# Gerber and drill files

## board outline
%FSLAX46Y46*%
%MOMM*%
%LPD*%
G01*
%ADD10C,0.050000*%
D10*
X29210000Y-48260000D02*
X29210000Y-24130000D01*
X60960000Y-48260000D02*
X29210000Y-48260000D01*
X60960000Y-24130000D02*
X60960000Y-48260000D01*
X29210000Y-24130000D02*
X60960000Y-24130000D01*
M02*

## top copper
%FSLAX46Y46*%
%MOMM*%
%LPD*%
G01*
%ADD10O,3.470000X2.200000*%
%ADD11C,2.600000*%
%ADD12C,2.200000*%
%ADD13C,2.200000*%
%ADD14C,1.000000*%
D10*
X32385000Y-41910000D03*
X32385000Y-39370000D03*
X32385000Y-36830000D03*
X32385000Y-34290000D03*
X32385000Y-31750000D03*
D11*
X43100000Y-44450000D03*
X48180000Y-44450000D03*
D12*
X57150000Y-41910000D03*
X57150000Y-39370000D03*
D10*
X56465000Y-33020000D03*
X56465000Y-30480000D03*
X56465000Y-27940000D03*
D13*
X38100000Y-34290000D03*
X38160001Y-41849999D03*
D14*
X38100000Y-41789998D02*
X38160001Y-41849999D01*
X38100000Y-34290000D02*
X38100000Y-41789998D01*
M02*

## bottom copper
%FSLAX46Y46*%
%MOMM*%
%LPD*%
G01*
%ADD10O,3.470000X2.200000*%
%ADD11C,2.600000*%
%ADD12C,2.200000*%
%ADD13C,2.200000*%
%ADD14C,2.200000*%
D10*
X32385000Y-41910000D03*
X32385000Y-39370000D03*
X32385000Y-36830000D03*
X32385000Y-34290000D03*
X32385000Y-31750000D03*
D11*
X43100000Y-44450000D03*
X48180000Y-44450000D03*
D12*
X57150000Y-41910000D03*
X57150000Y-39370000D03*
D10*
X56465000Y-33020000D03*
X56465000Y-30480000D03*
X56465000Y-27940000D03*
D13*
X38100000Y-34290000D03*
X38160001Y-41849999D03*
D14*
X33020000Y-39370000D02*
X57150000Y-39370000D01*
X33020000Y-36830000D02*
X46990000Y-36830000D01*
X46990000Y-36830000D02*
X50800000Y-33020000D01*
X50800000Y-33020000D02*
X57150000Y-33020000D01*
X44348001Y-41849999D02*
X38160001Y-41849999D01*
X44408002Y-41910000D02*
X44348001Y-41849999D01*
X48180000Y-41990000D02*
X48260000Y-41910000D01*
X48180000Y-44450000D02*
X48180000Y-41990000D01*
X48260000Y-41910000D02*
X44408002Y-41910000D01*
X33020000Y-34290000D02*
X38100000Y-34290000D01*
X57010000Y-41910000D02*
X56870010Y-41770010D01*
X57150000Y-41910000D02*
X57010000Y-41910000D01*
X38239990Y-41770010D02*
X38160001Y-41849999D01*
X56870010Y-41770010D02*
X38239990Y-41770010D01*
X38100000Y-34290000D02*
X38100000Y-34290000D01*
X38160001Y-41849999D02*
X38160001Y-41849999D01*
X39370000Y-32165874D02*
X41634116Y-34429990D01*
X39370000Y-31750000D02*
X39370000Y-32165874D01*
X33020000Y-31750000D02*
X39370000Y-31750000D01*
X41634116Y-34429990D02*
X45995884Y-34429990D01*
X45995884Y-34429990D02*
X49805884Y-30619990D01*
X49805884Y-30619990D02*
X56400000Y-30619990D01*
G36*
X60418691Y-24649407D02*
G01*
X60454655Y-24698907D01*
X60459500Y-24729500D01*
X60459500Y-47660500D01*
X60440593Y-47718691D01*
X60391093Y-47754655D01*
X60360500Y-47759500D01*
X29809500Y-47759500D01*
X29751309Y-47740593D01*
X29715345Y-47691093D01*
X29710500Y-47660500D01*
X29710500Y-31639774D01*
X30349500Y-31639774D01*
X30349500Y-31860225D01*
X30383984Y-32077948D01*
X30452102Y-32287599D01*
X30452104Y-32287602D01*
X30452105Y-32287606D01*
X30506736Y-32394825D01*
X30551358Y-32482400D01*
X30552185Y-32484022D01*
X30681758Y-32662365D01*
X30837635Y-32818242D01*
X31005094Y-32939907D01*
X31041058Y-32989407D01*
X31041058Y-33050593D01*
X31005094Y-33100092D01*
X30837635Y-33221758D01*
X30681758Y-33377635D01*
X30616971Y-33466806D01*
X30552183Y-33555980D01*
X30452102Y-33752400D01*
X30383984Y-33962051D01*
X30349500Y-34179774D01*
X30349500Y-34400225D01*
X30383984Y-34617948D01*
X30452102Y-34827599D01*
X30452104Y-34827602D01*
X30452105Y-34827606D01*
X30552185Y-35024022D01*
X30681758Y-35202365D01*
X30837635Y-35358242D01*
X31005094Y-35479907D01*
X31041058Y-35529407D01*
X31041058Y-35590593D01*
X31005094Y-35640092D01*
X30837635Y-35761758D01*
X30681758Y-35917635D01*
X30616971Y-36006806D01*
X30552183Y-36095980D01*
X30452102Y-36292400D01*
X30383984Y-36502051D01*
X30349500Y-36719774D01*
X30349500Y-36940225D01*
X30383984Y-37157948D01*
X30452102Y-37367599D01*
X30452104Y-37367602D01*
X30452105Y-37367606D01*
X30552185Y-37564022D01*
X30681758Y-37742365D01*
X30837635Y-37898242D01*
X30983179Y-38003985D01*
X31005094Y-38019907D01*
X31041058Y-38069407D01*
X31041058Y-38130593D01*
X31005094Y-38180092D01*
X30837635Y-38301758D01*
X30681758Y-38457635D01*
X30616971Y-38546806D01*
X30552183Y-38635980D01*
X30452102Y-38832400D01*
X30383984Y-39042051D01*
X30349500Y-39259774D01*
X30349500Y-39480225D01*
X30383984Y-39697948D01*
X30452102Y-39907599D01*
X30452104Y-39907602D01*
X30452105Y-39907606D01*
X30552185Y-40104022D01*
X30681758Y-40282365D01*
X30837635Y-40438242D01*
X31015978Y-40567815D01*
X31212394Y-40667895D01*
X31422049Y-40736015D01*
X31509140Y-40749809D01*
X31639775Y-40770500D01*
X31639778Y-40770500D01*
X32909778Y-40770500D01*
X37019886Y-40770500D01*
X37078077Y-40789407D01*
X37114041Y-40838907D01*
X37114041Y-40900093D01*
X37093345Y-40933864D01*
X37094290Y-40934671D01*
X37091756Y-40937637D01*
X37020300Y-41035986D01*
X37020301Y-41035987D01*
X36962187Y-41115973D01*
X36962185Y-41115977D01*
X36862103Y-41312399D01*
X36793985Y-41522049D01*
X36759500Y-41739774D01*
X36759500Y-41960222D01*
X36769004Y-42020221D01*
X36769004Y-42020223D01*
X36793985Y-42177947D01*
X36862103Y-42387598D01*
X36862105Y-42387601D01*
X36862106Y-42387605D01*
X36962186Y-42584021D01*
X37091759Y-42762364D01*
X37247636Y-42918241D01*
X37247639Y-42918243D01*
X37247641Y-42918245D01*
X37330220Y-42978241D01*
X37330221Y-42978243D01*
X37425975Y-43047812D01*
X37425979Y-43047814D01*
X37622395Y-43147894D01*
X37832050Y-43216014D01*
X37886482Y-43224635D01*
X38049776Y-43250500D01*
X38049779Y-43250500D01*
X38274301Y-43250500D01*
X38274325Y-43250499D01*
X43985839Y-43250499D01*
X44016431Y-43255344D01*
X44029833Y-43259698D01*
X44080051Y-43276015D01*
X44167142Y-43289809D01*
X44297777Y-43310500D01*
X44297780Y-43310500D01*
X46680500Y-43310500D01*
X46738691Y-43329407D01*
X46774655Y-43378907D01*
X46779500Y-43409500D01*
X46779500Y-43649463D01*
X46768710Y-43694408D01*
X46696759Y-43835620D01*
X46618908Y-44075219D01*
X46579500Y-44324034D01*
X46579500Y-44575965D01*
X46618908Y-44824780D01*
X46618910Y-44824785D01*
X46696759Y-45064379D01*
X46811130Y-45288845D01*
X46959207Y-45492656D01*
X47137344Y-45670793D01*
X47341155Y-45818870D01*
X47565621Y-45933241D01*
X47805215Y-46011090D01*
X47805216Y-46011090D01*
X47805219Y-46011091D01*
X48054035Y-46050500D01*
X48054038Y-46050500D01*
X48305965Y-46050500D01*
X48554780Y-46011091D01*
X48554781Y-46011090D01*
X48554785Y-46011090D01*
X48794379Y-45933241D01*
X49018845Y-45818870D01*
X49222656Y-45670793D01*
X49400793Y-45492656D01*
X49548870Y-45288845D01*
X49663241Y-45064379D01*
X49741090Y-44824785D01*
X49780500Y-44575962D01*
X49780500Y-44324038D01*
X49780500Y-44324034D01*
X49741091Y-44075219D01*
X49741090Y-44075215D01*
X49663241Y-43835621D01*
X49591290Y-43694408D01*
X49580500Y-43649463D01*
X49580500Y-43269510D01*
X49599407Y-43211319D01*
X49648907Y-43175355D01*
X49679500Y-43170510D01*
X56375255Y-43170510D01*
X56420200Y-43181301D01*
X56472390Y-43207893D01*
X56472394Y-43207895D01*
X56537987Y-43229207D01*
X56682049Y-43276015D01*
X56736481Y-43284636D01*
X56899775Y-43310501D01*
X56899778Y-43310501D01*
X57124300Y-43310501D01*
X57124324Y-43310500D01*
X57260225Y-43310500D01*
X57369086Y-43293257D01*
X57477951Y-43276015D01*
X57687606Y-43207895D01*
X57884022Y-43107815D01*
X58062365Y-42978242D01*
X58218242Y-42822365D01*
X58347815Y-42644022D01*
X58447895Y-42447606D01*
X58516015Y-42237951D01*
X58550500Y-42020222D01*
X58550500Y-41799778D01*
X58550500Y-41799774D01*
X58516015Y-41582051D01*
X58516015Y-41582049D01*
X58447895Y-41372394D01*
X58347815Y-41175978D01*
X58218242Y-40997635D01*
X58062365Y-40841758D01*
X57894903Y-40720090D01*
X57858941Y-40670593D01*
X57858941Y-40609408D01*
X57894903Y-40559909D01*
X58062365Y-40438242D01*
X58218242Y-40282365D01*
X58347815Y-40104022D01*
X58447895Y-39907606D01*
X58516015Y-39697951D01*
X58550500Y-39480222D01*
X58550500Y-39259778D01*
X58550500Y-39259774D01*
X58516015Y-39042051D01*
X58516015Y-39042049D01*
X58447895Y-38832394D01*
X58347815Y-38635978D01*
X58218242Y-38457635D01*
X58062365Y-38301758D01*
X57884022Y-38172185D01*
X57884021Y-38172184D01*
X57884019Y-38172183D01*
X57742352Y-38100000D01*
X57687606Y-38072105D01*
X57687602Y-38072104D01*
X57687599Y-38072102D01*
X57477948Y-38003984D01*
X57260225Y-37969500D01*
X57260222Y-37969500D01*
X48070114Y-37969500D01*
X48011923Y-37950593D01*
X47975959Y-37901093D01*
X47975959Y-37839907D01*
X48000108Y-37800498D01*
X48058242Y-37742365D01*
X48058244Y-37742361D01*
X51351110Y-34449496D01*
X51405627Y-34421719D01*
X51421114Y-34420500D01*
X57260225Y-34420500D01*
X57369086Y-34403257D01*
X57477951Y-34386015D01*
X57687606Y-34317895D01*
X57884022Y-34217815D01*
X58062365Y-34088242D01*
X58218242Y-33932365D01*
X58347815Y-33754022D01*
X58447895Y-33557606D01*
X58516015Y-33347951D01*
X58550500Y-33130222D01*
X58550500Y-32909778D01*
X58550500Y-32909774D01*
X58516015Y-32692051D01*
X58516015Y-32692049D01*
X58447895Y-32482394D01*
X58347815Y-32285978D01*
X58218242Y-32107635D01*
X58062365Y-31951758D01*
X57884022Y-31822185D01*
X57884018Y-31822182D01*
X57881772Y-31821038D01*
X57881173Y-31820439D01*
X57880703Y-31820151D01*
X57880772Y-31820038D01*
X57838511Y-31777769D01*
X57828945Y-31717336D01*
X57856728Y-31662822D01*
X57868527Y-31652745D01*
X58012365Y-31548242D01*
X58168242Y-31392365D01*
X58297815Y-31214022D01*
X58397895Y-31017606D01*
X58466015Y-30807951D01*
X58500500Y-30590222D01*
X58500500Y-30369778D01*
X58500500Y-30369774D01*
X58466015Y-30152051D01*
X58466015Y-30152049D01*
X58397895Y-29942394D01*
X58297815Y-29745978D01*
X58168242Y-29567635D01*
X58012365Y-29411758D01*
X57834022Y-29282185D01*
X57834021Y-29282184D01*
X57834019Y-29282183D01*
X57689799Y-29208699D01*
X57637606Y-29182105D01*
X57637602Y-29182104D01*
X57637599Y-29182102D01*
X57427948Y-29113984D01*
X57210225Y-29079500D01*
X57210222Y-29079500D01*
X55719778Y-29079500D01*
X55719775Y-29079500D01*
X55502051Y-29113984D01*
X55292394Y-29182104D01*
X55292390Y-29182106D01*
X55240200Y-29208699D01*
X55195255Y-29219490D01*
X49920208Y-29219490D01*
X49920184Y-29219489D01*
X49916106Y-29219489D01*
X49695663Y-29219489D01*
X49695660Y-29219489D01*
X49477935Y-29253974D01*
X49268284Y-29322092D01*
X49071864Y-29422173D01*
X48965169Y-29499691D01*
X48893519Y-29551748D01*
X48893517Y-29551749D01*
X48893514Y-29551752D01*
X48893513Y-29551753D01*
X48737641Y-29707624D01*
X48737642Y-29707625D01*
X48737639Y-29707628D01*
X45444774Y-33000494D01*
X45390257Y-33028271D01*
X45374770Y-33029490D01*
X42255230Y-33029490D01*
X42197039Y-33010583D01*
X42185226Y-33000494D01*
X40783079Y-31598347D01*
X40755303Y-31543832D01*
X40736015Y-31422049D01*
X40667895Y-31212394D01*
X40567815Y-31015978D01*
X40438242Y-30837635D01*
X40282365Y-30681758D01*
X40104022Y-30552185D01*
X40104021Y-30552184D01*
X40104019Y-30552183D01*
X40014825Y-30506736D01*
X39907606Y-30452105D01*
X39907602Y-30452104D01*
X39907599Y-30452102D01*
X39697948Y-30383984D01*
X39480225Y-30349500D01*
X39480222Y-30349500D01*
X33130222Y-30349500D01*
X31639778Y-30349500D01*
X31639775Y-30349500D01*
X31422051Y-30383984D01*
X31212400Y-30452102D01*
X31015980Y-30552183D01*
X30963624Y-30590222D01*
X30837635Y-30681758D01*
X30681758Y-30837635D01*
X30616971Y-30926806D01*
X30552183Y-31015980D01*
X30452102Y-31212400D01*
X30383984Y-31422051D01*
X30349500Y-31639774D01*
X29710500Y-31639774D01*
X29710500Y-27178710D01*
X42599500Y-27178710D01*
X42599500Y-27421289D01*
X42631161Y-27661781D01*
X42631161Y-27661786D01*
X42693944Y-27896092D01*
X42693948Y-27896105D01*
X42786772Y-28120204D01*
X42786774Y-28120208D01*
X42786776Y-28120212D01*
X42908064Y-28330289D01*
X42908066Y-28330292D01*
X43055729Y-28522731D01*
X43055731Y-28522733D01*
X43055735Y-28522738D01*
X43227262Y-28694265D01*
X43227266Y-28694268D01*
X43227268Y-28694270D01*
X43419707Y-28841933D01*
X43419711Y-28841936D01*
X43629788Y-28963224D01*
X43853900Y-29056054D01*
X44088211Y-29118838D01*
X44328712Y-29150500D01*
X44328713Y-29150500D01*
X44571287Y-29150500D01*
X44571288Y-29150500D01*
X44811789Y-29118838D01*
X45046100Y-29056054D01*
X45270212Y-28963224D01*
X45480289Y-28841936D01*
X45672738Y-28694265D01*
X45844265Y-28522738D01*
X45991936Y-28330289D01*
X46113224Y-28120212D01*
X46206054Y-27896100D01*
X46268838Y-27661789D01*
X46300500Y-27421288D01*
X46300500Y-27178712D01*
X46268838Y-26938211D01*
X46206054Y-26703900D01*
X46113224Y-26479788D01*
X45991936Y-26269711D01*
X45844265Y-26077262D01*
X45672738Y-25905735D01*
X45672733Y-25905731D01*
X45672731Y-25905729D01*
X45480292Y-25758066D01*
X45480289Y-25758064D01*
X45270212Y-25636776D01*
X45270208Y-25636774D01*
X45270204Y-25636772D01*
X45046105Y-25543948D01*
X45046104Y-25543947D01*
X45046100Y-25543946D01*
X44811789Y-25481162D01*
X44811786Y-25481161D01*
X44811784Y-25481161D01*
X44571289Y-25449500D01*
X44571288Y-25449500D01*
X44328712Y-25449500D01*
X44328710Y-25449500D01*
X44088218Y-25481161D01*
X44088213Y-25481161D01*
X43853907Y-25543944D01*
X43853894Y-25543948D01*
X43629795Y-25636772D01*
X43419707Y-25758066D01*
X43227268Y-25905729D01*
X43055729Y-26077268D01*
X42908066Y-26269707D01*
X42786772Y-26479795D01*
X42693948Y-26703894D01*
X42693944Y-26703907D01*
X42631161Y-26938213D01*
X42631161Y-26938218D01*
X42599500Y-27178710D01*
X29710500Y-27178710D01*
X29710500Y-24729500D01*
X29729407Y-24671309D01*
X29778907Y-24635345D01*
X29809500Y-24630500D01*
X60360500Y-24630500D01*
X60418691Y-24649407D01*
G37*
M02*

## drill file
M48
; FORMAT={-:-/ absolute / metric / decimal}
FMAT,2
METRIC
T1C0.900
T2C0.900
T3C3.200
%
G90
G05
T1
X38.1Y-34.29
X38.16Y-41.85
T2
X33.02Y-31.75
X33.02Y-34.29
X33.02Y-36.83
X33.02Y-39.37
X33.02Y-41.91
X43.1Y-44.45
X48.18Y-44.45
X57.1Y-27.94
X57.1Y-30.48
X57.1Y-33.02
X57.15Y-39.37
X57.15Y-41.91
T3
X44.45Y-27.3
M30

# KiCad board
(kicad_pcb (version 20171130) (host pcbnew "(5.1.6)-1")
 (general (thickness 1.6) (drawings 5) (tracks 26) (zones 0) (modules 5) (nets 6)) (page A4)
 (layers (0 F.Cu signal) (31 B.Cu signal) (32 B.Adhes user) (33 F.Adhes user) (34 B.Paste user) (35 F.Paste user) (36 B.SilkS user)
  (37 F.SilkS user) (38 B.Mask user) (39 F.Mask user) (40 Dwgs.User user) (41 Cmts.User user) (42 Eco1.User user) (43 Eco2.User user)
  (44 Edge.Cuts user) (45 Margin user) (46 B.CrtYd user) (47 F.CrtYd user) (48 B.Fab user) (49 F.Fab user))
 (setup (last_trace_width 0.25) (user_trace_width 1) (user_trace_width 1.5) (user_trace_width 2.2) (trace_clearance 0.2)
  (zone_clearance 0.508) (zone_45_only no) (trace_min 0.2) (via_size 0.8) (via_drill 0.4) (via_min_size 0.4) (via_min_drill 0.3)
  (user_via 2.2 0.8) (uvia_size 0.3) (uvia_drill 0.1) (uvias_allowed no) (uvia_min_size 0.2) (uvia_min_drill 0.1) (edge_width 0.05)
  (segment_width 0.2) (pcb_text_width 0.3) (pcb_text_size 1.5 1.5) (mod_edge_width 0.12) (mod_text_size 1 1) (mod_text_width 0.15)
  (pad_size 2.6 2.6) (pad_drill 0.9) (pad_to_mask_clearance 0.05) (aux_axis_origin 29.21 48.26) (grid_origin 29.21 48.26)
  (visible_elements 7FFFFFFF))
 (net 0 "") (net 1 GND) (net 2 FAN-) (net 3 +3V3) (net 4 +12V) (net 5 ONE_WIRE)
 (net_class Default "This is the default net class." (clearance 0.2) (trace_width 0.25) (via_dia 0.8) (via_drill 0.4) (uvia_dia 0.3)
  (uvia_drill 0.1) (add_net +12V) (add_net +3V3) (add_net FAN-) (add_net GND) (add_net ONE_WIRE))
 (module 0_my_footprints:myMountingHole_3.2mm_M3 (layer F.Cu) (at 44.45 27.3)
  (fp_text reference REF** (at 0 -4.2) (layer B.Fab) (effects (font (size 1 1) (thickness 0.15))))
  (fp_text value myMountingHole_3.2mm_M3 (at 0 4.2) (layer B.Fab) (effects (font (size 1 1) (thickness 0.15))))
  (pad "" np_thru_hole circle (at 0 0) (size 3.2 3.2) (drill 3.2) (layers *.Cu *.Mask)))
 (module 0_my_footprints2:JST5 (layer F.Cu) (at 33.02 41.91 90)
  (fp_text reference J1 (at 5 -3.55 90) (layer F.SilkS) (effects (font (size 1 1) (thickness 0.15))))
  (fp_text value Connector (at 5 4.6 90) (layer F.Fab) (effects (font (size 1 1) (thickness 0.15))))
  (pad 1 thru_hole oval (at 0 0 90) (size 2.2 3.47) (drill 0.9 (offset 0 -0.635)) (layers *.Cu *.Mask) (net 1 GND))
  (pad 2 thru_hole oval (at 2.54 0 90) (size 2.2 3.47) (drill 0.9 (offset 0 -0.635)) (layers *.Cu *.Mask) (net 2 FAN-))
  (pad 3 thru_hole oval (at 5.08 0 90) (size 2.2 3.47) (drill 0.9 (offset 0 -0.635)) (layers *.Cu *.Mask) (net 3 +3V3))
  (pad 4 thru_hole oval (at 7.62 0 90) (size 2.2 3.47) (drill 0.9 (offset 0 -0.635)) (layers *.Cu *.Mask) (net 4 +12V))
  (pad 5 thru_hole oval (at 10.16 0 90) (size 2.2 3.47) (drill 0.9 (offset 0 -0.635)) (layers *.Cu *.Mask) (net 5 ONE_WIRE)))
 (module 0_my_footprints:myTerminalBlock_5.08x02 (layer F.Cu) (at 43.1 44.45)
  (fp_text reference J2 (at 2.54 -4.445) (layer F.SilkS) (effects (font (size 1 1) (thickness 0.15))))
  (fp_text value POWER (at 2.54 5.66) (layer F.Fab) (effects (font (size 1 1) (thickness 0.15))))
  (pad 1 thru_hole circle (at 0 0) (size 2.6 2.6) (drill 0.9) (layers *.Cu *.Mask) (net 1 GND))
  (pad 2 thru_hole circle (at 5.08 0) (size 2.6 2.6) (drill 0.9) (layers *.Cu *.Mask) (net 4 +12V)))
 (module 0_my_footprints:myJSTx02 (layer F.Cu) (at 57.15 41.91 90)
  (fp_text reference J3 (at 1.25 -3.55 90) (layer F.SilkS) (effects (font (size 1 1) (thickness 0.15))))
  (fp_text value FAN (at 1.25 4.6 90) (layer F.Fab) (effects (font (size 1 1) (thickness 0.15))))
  (pad 1 thru_hole circle (at 0 0 90) (size 2.2 2.2) (drill 0.9) (layers *.Cu *.Mask) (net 4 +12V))
  (pad 2 thru_hole circle (at 2.54 0 90) (size 2.2 2.2) (drill 0.9) (layers *.Cu *.Mask) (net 2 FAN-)))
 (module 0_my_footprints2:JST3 (layer F.Cu) (at 57.1 33.02 90)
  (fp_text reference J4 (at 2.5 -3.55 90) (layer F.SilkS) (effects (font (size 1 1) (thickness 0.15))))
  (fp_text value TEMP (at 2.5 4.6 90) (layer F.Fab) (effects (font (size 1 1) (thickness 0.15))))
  (pad 1 thru_hole oval (at 0 0 90) (size 2.2 3.47) (drill 0.9 (offset 0 -0.635)) (layers *.Cu *.Mask) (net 3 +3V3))
  (pad 2 thru_hole oval (at 2.54 0 90) (size 2.2 3.47) (drill 0.9 (offset 0 -0.635)) (layers *.Cu *.Mask) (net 5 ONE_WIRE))
  (pad 3 thru_hole oval (at 5.08 0 90) (size 2.2 3.47) (drill 0.9 (offset 0 -0.635)) (layers *.Cu *.Mask) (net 1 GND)))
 (gr_line (start 29.21 48.26) (end 29.21 24.13) (layer Edge.Cuts) (width 0.05))
 (gr_line (start 60.96 48.26) (end 29.21 48.26) (layer Edge.Cuts) (width 0.05))
 (gr_line (start 60.96 24.13) (end 60.96 48.26) (layer Edge.Cuts) (width 0.05))
 (gr_line (start 29.21 24.13) (end 60.96 24.13) (layer Edge.Cuts) (width 0.05))
 (segment (start 33.02 39.37) (end 57.15 39.37) (width 2.2) (layer B.Cu) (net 2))
 (segment (start 33.02 36.83) (end 46.99 36.83) (width 2.2) (layer B.Cu) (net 3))
 (segment (start 46.99 36.83) (end 50.8 33.02) (width 2.2) (layer B.Cu) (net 3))
 (segment (start 50.8 33.02) (end 57.15 33.02) (width 2.2) (layer B.Cu) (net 3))
 (segment (start 44.348001 41.849999) (end 38.160001 41.849999) (width 2.2) (layer B.Cu) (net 4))
 (segment (start 44.408002 41.91) (end 44.348001 41.849999) (width 2.2) (layer B.Cu) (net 4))
 (segment (start 48.18 41.99) (end 48.26 41.91) (width 2.2) (layer B.Cu) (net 4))
 (segment (start 48.18 44.45) (end 48.18 41.99) (width 2.2) (layer B.Cu) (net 4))
 (segment (start 48.26 41.91) (end 44.408002 41.91) (width 2.2) (layer B.Cu) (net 4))
 (segment (start 33.02 34.29) (end 38.1 34.29) (width 2.2) (layer B.Cu) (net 4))
 (segment (start 57.01 41.91) (end 56.87001 41.77001) (width 2.2) (layer B.Cu) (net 4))
 (segment (start 57.15 41.91) (end 57.01 41.91) (width 2.2) (layer B.Cu) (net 4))
 (segment (start 38.23999 41.77001) (end 38.160001 41.849999) (width 2.2) (layer B.Cu) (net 4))
 (segment (start 56.87001 41.77001) (end 38.23999 41.77001) (width 2.2) (layer B.Cu) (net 4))
 (segment (start 38.1 34.29) (end 38.1 34.29) (width 2.2) (layer B.Cu) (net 4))
 (via (at 38.1 34.29) (size 2.2) (drill 0.9) (layers F.Cu B.Cu) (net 4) (status 1000000))
 (segment (start 38.160001 41.849999) (end 38.160001 41.849999) (width 2.2) (layer B.Cu) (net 4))
 (via (at 38.160001 41.849999) (size 2.2) (drill 0.9) (layers F.Cu B.Cu) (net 4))
 (segment (start 38.1 41.789998) (end 38.160001 41.849999) (width 1) (layer F.Cu) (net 4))
 (segment (start 38.1 34.29) (end 38.1 41.789998) (width 1) (layer F.Cu) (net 4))
 (segment (start 39.37 32.165874) (end 41.634116 34.42999) (width 2.2) (layer B.Cu) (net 5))
 (segment (start 39.37 31.75) (end 39.37 32.165874) (width 2.2) (layer B.Cu) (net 5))
 (segment (start 33.02 31.75) (end 39.37 31.75) (width 2.2) (layer B.Cu) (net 5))
 (segment (start 41.634116 34.42999) (end 45.995884 34.42999) (width 2.2) (layer B.Cu) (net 5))
 (segment (start 45.995884 34.42999) (end 49.805884 30.61999) (width 2.2) (layer B.Cu) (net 5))
 (segment (start 49.805884 30.61999) (end 56.4 30.61999) (width 2.2) (layer B.Cu) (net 5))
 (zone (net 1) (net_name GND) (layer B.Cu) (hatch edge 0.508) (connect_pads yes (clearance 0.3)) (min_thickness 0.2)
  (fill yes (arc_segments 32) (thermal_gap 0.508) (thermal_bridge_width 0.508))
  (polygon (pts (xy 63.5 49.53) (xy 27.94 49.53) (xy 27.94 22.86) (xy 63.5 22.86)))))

